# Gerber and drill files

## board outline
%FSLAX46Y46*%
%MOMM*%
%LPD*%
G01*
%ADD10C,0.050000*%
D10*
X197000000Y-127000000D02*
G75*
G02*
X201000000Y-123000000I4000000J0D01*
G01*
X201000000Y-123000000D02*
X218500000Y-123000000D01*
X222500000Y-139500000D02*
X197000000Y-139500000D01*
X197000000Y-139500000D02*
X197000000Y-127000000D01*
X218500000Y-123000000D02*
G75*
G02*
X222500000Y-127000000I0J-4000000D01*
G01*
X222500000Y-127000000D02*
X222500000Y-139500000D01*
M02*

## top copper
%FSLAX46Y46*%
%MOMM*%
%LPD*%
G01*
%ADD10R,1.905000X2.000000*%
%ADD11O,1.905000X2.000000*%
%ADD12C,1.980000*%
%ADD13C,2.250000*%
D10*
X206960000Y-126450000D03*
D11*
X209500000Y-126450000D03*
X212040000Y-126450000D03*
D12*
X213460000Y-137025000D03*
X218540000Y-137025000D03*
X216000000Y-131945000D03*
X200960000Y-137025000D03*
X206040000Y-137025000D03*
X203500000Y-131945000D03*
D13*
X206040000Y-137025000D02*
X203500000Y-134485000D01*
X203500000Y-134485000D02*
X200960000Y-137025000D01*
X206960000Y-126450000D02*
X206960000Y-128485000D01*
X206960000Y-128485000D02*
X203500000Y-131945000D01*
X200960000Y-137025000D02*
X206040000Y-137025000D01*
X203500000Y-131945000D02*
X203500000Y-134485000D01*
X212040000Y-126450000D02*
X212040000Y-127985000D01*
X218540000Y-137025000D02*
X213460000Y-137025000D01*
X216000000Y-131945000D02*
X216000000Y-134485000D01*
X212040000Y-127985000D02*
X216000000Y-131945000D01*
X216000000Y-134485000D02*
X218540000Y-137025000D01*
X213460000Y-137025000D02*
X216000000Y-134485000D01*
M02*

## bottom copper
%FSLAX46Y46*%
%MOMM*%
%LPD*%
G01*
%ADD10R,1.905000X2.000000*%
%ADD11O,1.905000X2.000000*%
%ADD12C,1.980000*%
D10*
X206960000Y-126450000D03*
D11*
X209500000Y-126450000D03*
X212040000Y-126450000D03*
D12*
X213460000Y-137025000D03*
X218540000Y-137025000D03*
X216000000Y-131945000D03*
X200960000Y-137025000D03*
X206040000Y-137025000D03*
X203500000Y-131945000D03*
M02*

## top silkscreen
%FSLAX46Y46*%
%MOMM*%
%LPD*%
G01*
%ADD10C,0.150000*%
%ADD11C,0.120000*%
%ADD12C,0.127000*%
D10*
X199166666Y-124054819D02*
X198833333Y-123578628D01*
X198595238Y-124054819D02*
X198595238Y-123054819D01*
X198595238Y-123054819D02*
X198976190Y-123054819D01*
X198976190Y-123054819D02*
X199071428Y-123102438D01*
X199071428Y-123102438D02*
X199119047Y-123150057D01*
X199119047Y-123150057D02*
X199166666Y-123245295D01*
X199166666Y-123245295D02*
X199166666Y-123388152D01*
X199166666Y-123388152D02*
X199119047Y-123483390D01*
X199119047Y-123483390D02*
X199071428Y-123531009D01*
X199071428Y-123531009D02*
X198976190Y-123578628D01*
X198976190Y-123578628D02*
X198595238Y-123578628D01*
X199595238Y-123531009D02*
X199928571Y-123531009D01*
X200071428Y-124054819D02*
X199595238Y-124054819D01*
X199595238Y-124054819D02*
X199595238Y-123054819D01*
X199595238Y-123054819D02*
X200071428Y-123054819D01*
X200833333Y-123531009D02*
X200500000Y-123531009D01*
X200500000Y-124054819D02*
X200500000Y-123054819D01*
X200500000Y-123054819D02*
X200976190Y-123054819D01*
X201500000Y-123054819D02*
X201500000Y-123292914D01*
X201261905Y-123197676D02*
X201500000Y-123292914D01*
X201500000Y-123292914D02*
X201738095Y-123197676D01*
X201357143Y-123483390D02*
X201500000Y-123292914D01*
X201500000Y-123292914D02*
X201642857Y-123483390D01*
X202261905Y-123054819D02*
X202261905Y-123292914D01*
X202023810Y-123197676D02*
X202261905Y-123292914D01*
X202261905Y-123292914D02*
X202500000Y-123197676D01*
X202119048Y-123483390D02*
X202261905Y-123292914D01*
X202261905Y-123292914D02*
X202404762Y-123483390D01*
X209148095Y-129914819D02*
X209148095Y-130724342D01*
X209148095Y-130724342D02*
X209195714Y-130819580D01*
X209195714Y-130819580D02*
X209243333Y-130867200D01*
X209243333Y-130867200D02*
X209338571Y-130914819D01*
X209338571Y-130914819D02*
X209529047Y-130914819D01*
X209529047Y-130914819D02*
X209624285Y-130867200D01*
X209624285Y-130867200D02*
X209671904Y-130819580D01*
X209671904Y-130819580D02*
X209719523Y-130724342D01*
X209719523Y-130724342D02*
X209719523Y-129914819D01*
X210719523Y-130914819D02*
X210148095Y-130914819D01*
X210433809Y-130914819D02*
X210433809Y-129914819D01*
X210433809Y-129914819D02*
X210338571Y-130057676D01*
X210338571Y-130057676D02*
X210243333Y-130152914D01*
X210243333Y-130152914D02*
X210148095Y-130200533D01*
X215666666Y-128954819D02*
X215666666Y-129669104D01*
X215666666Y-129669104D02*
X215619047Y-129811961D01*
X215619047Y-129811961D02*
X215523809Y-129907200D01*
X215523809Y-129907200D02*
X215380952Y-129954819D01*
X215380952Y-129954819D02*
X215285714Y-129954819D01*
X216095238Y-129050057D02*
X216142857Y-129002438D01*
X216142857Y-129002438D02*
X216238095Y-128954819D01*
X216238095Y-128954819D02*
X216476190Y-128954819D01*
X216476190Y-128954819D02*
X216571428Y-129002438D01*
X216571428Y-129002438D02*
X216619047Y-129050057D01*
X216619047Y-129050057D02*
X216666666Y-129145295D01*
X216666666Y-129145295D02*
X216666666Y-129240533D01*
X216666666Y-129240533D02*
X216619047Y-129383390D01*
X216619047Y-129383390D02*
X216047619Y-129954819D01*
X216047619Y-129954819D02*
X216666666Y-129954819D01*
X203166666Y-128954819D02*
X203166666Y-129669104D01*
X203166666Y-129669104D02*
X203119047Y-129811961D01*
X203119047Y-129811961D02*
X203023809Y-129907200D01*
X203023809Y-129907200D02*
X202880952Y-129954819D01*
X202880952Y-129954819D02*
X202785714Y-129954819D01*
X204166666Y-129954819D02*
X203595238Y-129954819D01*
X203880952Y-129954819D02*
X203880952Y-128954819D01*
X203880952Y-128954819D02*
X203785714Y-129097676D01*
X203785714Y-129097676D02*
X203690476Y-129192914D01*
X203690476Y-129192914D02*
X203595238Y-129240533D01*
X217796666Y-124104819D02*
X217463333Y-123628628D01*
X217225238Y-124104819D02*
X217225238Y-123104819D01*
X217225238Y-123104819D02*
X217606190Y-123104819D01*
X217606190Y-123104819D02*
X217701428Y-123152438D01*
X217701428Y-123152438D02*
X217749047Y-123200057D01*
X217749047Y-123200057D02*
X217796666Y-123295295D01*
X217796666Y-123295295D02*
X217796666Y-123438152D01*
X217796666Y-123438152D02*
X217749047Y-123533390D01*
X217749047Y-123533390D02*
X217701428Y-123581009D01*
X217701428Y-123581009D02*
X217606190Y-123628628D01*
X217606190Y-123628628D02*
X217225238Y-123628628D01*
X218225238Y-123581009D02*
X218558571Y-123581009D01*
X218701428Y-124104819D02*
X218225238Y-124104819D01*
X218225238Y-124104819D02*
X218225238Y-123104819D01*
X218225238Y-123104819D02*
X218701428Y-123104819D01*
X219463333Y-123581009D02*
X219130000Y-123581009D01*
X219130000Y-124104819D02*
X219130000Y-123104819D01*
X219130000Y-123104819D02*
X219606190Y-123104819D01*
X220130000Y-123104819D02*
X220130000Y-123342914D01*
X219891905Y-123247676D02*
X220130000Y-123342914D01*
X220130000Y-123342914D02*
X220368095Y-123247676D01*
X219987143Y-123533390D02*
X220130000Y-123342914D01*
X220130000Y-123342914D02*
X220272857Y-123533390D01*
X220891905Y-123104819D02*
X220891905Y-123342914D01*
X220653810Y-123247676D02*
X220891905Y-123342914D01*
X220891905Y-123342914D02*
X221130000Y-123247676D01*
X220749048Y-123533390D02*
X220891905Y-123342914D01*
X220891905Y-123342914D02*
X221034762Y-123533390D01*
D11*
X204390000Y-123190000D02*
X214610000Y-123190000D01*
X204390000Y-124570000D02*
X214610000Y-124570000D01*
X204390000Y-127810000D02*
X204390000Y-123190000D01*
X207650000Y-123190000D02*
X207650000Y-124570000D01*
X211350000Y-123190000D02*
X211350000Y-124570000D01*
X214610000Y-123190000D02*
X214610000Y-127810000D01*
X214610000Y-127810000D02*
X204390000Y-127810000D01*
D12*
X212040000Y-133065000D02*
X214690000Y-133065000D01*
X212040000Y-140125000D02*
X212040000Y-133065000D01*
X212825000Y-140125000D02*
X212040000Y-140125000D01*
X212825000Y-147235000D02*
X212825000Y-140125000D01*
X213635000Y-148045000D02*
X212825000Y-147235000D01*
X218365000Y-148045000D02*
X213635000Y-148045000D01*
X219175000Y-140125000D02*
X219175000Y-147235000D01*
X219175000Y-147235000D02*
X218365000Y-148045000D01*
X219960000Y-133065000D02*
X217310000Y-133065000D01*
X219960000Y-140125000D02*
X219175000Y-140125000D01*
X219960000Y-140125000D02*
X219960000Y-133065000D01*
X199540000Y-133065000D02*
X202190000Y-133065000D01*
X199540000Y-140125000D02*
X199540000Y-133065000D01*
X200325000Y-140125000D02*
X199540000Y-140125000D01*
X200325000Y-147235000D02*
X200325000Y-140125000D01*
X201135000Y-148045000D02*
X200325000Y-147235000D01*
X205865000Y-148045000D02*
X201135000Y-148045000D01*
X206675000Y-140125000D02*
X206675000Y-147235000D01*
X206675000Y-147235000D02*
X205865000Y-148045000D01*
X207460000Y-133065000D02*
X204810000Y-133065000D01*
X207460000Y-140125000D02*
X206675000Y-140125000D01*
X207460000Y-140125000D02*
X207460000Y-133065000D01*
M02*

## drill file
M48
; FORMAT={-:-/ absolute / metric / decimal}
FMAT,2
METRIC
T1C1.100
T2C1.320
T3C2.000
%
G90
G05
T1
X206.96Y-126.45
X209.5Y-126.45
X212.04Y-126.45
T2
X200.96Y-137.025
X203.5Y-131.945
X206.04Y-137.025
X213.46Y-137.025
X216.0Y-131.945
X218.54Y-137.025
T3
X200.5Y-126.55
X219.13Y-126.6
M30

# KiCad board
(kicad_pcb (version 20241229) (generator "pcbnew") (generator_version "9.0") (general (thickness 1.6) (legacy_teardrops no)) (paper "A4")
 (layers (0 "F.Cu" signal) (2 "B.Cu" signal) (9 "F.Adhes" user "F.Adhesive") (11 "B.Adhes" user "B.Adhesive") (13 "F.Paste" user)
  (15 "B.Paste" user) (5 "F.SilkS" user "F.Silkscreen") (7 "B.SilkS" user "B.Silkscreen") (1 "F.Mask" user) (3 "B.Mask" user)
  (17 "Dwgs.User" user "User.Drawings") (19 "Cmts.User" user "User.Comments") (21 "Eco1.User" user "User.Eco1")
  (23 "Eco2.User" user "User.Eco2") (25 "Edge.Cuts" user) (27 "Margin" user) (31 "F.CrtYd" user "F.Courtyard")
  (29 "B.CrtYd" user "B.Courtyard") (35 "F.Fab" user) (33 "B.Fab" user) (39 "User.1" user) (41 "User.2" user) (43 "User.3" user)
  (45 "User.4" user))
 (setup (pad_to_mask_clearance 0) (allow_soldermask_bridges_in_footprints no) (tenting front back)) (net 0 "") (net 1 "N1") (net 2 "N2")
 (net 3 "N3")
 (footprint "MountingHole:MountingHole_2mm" (layer "F.Cu") (at 200.5 126.55)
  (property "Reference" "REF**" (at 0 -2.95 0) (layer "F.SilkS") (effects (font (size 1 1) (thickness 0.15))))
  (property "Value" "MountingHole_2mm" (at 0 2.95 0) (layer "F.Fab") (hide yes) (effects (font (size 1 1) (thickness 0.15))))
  (pad "" np_thru_hole circle (at 0 0) (size 2 2) (drill 2) (layers "*.Cu" "*.Mask")))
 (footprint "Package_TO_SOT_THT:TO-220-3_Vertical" (layer "F.Cu") (at 206.96 126.45)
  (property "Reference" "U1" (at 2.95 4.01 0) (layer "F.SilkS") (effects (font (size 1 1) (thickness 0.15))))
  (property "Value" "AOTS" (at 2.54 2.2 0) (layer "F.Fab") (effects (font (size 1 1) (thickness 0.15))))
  (fp_line (start -2.57 -3.26) (end 7.65 -3.26) (stroke (width 0.12) (type solid)) (layer "F.SilkS"))
  (fp_line (start -2.57 -1.88) (end 7.65 -1.88) (stroke (width 0.12) (type solid)) (layer "F.SilkS"))
  (fp_line (start -2.57 1.36) (end -2.57 -3.26) (stroke (width 0.12) (type solid)) (layer "F.SilkS"))
  (fp_line (start 0.69 -3.26) (end 0.69 -1.88) (stroke (width 0.12) (type solid)) (layer "F.SilkS"))
  (fp_line (start 4.39 -3.26) (end 4.39 -1.88) (stroke (width 0.12) (type solid)) (layer "F.SilkS"))
  (fp_line (start 7.65 -3.26) (end 7.65 1.36) (stroke (width 0.12) (type solid)) (layer "F.SilkS"))
  (fp_line (start 7.65 1.36) (end -2.57 1.36) (stroke (width 0.12) (type solid)) (layer "F.SilkS"))
  (pad "1" thru_hole rect (at 0 0) (size 1.905 2) (drill 1.1) (layers "*.Cu" "*.Mask") (remove_unused_layers no) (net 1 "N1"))
  (pad "2" thru_hole oval (at 2.54 0) (size 1.905 2) (drill 1.1) (layers "*.Cu" "*.Mask") (remove_unused_layers no) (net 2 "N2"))
  (pad "3" thru_hole oval (at 5.08 0) (size 1.905 2) (drill 1.1) (layers "*.Cu" "*.Mask") (remove_unused_layers no) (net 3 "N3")))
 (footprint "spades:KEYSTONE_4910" (layer "F.Cu") (at 216 137.025 90)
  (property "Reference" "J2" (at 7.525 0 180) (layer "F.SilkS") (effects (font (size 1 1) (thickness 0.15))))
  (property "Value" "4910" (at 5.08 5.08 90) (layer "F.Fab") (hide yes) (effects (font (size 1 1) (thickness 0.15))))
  (fp_line (start 3.96 -3.96) (end 3.96 -1.31) (stroke (width 0.127) (type solid)) (layer "F.SilkS"))
  (fp_line (start -3.1 -3.96) (end 3.96 -3.96) (stroke (width 0.127) (type solid)) (layer "F.SilkS"))
  (fp_line (start -3.1 -3.175) (end -3.1 -3.96) (stroke (width 0.127) (type solid)) (layer "F.SilkS"))
  (fp_line (start -10.21 -3.175) (end -3.1 -3.175) (stroke (width 0.127) (type solid)) (layer "F.SilkS"))
  (fp_line (start -11.02 -2.365) (end -10.21 -3.175) (stroke (width 0.127) (type solid)) (layer "F.SilkS"))
  (fp_line (start -11.02 2.365) (end -11.02 -2.365) (stroke (width 0.127) (type solid)) (layer "F.SilkS"))
  (fp_line (start -3.1 3.175) (end -10.21 3.175) (stroke (width 0.127) (type solid)) (layer "F.SilkS"))
  (fp_line (start -10.21 3.175) (end -11.02 2.365) (stroke (width 0.127) (type solid)) (layer "F.SilkS"))
  (fp_line (start 3.96 3.96) (end 3.96 1.31) (stroke (width 0.127) (type solid)) (layer "F.SilkS"))
  (fp_line (start -3.1 3.96) (end -3.1 3.175) (stroke (width 0.127) (type solid)) (layer "F.SilkS"))
  (fp_line (start -3.1 3.96) (end 3.96 3.96) (stroke (width 0.127) (type solid)) (layer "F.SilkS"))
  (pad "1_1" thru_hole circle (at 0 -2.54 90) (size 1.98 1.98) (drill 1.32) (layers "*.Cu" "*.Mask") (remove_unused_layers no) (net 3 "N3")
   (solder_mask_margin 0.102))
  (pad "1_2" thru_hole circle (at 0 2.54 90) (size 1.98 1.98) (drill 1.32) (layers "*.Cu" "*.Mask") (remove_unused_layers no) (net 3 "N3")
   (solder_mask_margin 0.102))
  (pad "1_3" thru_hole circle (at 5.08 0 90) (size 1.98 1.98) (drill 1.32) (layers "*.Cu" "*.Mask") (remove_unused_layers no) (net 3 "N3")
   (solder_mask_margin 0.102)))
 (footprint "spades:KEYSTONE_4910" (layer "F.Cu") (at 203.5 137.025 90)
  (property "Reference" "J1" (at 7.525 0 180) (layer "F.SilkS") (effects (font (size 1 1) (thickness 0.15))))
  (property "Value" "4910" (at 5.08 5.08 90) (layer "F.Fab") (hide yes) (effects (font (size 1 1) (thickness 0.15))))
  (fp_line (start 3.96 -3.96) (end 3.96 -1.31) (stroke (width 0.127) (type solid)) (layer "F.SilkS"))
  (fp_line (start -3.1 -3.96) (end 3.96 -3.96) (stroke (width 0.127) (type solid)) (layer "F.SilkS"))
  (fp_line (start -3.1 -3.175) (end -3.1 -3.96) (stroke (width 0.127) (type solid)) (layer "F.SilkS"))
  (fp_line (start -10.21 -3.175) (end -3.1 -3.175) (stroke (width 0.127) (type solid)) (layer "F.SilkS"))
  (fp_line (start -11.02 -2.365) (end -10.21 -3.175) (stroke (width 0.127) (type solid)) (layer "F.SilkS"))
  (fp_line (start -11.02 2.365) (end -11.02 -2.365) (stroke (width 0.127) (type solid)) (layer "F.SilkS"))
  (fp_line (start -3.1 3.175) (end -10.21 3.175) (stroke (width 0.127) (type solid)) (layer "F.SilkS"))
  (fp_line (start -10.21 3.175) (end -11.02 2.365) (stroke (width 0.127) (type solid)) (layer "F.SilkS"))
  (fp_line (start 3.96 3.96) (end 3.96 1.31) (stroke (width 0.127) (type solid)) (layer "F.SilkS"))
  (fp_line (start -3.1 3.96) (end -3.1 3.175) (stroke (width 0.127) (type solid)) (layer "F.SilkS"))
  (fp_line (start -3.1 3.96) (end 3.96 3.96) (stroke (width 0.127) (type solid)) (layer "F.SilkS"))
  (pad "1_1" thru_hole circle (at 0 -2.54 90) (size 1.98 1.98) (drill 1.32) (layers "*.Cu" "*.Mask") (remove_unused_layers no) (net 1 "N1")
   (solder_mask_margin 0.102))
  (pad "1_2" thru_hole circle (at 0 2.54 90) (size 1.98 1.98) (drill 1.32) (layers "*.Cu" "*.Mask") (remove_unused_layers no) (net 1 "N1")
   (solder_mask_margin 0.102))
  (pad "1_3" thru_hole circle (at 5.08 0 90) (size 1.98 1.98) (drill 1.32) (layers "*.Cu" "*.Mask") (remove_unused_layers no) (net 1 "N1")
   (solder_mask_margin 0.102)))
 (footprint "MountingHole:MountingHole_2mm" (layer "F.Cu") (at 219.13 126.6)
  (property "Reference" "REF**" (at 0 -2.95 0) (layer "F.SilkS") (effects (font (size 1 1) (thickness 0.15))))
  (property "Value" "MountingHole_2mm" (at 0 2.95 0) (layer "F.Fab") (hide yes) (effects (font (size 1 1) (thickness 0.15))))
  (pad "" np_thru_hole circle (at 0 0) (size 2 2) (drill 2) (layers "*.Cu" "*.Mask")))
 (gr_arc (start 197 127) (mid 198.171573 124.171573) (end 201 123) (stroke (width 0.05) (type default)) (layer "Edge.Cuts"))
 (gr_line (start 201 123) (end 218.5 123) (stroke (width 0.05) (type default)) (layer "Edge.Cuts"))
 (gr_line (start 222.5 139.5) (end 197 139.5) (stroke (width 0.05) (type default)) (layer "Edge.Cuts"))
 (gr_line (start 197 139.5) (end 197 127) (stroke (width 0.05) (type default)) (layer "Edge.Cuts"))
 (gr_arc (start 218.5 123) (mid 221.328427 124.171573) (end 222.5 127) (stroke (width 0.05) (type default)) (layer "Edge.Cuts"))
 (gr_line (start 222.5 127) (end 222.5 139.5) (stroke (width 0.05) (type default)) (layer "Edge.Cuts"))
 (segment (start 206.04 137.025) (end 203.5 134.485) (width 2.25) (layer "F.Cu") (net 1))
 (segment (start 203.5 134.485) (end 200.96 137.025) (width 2.25) (layer "F.Cu") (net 1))
 (segment (start 206.96 126.45) (end 206.96 128.485) (width 2.25) (layer "F.Cu") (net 1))
 (segment (start 206.96 128.485) (end 203.5 131.945) (width 2.25) (layer "F.Cu") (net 1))
 (segment (start 200.96 137.025) (end 206.04 137.025) (width 2.25) (layer "F.Cu") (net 1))
 (segment (start 203.5 131.945) (end 203.5 134.485) (width 2.25) (layer "F.Cu") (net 1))
 (segment (start 212.04 126.45) (end 212.04 127.985) (width 2.25) (layer "F.Cu") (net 3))
 (segment (start 218.54 137.025) (end 213.46 137.025) (width 2.25) (layer "F.Cu") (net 3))
 (segment (start 216 131.945) (end 216 134.485) (width 2.25) (layer "F.Cu") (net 3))
 (segment (start 212.04 127.985) (end 216 131.945) (width 2.25) (layer "F.Cu") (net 3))
 (segment (start 216 134.485) (end 218.54 137.025) (width 2.25) (layer "F.Cu") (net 3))
 (segment (start 213.46 137.025) (end 216 134.485) (width 2.25) (layer "F.Cu") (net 3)))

